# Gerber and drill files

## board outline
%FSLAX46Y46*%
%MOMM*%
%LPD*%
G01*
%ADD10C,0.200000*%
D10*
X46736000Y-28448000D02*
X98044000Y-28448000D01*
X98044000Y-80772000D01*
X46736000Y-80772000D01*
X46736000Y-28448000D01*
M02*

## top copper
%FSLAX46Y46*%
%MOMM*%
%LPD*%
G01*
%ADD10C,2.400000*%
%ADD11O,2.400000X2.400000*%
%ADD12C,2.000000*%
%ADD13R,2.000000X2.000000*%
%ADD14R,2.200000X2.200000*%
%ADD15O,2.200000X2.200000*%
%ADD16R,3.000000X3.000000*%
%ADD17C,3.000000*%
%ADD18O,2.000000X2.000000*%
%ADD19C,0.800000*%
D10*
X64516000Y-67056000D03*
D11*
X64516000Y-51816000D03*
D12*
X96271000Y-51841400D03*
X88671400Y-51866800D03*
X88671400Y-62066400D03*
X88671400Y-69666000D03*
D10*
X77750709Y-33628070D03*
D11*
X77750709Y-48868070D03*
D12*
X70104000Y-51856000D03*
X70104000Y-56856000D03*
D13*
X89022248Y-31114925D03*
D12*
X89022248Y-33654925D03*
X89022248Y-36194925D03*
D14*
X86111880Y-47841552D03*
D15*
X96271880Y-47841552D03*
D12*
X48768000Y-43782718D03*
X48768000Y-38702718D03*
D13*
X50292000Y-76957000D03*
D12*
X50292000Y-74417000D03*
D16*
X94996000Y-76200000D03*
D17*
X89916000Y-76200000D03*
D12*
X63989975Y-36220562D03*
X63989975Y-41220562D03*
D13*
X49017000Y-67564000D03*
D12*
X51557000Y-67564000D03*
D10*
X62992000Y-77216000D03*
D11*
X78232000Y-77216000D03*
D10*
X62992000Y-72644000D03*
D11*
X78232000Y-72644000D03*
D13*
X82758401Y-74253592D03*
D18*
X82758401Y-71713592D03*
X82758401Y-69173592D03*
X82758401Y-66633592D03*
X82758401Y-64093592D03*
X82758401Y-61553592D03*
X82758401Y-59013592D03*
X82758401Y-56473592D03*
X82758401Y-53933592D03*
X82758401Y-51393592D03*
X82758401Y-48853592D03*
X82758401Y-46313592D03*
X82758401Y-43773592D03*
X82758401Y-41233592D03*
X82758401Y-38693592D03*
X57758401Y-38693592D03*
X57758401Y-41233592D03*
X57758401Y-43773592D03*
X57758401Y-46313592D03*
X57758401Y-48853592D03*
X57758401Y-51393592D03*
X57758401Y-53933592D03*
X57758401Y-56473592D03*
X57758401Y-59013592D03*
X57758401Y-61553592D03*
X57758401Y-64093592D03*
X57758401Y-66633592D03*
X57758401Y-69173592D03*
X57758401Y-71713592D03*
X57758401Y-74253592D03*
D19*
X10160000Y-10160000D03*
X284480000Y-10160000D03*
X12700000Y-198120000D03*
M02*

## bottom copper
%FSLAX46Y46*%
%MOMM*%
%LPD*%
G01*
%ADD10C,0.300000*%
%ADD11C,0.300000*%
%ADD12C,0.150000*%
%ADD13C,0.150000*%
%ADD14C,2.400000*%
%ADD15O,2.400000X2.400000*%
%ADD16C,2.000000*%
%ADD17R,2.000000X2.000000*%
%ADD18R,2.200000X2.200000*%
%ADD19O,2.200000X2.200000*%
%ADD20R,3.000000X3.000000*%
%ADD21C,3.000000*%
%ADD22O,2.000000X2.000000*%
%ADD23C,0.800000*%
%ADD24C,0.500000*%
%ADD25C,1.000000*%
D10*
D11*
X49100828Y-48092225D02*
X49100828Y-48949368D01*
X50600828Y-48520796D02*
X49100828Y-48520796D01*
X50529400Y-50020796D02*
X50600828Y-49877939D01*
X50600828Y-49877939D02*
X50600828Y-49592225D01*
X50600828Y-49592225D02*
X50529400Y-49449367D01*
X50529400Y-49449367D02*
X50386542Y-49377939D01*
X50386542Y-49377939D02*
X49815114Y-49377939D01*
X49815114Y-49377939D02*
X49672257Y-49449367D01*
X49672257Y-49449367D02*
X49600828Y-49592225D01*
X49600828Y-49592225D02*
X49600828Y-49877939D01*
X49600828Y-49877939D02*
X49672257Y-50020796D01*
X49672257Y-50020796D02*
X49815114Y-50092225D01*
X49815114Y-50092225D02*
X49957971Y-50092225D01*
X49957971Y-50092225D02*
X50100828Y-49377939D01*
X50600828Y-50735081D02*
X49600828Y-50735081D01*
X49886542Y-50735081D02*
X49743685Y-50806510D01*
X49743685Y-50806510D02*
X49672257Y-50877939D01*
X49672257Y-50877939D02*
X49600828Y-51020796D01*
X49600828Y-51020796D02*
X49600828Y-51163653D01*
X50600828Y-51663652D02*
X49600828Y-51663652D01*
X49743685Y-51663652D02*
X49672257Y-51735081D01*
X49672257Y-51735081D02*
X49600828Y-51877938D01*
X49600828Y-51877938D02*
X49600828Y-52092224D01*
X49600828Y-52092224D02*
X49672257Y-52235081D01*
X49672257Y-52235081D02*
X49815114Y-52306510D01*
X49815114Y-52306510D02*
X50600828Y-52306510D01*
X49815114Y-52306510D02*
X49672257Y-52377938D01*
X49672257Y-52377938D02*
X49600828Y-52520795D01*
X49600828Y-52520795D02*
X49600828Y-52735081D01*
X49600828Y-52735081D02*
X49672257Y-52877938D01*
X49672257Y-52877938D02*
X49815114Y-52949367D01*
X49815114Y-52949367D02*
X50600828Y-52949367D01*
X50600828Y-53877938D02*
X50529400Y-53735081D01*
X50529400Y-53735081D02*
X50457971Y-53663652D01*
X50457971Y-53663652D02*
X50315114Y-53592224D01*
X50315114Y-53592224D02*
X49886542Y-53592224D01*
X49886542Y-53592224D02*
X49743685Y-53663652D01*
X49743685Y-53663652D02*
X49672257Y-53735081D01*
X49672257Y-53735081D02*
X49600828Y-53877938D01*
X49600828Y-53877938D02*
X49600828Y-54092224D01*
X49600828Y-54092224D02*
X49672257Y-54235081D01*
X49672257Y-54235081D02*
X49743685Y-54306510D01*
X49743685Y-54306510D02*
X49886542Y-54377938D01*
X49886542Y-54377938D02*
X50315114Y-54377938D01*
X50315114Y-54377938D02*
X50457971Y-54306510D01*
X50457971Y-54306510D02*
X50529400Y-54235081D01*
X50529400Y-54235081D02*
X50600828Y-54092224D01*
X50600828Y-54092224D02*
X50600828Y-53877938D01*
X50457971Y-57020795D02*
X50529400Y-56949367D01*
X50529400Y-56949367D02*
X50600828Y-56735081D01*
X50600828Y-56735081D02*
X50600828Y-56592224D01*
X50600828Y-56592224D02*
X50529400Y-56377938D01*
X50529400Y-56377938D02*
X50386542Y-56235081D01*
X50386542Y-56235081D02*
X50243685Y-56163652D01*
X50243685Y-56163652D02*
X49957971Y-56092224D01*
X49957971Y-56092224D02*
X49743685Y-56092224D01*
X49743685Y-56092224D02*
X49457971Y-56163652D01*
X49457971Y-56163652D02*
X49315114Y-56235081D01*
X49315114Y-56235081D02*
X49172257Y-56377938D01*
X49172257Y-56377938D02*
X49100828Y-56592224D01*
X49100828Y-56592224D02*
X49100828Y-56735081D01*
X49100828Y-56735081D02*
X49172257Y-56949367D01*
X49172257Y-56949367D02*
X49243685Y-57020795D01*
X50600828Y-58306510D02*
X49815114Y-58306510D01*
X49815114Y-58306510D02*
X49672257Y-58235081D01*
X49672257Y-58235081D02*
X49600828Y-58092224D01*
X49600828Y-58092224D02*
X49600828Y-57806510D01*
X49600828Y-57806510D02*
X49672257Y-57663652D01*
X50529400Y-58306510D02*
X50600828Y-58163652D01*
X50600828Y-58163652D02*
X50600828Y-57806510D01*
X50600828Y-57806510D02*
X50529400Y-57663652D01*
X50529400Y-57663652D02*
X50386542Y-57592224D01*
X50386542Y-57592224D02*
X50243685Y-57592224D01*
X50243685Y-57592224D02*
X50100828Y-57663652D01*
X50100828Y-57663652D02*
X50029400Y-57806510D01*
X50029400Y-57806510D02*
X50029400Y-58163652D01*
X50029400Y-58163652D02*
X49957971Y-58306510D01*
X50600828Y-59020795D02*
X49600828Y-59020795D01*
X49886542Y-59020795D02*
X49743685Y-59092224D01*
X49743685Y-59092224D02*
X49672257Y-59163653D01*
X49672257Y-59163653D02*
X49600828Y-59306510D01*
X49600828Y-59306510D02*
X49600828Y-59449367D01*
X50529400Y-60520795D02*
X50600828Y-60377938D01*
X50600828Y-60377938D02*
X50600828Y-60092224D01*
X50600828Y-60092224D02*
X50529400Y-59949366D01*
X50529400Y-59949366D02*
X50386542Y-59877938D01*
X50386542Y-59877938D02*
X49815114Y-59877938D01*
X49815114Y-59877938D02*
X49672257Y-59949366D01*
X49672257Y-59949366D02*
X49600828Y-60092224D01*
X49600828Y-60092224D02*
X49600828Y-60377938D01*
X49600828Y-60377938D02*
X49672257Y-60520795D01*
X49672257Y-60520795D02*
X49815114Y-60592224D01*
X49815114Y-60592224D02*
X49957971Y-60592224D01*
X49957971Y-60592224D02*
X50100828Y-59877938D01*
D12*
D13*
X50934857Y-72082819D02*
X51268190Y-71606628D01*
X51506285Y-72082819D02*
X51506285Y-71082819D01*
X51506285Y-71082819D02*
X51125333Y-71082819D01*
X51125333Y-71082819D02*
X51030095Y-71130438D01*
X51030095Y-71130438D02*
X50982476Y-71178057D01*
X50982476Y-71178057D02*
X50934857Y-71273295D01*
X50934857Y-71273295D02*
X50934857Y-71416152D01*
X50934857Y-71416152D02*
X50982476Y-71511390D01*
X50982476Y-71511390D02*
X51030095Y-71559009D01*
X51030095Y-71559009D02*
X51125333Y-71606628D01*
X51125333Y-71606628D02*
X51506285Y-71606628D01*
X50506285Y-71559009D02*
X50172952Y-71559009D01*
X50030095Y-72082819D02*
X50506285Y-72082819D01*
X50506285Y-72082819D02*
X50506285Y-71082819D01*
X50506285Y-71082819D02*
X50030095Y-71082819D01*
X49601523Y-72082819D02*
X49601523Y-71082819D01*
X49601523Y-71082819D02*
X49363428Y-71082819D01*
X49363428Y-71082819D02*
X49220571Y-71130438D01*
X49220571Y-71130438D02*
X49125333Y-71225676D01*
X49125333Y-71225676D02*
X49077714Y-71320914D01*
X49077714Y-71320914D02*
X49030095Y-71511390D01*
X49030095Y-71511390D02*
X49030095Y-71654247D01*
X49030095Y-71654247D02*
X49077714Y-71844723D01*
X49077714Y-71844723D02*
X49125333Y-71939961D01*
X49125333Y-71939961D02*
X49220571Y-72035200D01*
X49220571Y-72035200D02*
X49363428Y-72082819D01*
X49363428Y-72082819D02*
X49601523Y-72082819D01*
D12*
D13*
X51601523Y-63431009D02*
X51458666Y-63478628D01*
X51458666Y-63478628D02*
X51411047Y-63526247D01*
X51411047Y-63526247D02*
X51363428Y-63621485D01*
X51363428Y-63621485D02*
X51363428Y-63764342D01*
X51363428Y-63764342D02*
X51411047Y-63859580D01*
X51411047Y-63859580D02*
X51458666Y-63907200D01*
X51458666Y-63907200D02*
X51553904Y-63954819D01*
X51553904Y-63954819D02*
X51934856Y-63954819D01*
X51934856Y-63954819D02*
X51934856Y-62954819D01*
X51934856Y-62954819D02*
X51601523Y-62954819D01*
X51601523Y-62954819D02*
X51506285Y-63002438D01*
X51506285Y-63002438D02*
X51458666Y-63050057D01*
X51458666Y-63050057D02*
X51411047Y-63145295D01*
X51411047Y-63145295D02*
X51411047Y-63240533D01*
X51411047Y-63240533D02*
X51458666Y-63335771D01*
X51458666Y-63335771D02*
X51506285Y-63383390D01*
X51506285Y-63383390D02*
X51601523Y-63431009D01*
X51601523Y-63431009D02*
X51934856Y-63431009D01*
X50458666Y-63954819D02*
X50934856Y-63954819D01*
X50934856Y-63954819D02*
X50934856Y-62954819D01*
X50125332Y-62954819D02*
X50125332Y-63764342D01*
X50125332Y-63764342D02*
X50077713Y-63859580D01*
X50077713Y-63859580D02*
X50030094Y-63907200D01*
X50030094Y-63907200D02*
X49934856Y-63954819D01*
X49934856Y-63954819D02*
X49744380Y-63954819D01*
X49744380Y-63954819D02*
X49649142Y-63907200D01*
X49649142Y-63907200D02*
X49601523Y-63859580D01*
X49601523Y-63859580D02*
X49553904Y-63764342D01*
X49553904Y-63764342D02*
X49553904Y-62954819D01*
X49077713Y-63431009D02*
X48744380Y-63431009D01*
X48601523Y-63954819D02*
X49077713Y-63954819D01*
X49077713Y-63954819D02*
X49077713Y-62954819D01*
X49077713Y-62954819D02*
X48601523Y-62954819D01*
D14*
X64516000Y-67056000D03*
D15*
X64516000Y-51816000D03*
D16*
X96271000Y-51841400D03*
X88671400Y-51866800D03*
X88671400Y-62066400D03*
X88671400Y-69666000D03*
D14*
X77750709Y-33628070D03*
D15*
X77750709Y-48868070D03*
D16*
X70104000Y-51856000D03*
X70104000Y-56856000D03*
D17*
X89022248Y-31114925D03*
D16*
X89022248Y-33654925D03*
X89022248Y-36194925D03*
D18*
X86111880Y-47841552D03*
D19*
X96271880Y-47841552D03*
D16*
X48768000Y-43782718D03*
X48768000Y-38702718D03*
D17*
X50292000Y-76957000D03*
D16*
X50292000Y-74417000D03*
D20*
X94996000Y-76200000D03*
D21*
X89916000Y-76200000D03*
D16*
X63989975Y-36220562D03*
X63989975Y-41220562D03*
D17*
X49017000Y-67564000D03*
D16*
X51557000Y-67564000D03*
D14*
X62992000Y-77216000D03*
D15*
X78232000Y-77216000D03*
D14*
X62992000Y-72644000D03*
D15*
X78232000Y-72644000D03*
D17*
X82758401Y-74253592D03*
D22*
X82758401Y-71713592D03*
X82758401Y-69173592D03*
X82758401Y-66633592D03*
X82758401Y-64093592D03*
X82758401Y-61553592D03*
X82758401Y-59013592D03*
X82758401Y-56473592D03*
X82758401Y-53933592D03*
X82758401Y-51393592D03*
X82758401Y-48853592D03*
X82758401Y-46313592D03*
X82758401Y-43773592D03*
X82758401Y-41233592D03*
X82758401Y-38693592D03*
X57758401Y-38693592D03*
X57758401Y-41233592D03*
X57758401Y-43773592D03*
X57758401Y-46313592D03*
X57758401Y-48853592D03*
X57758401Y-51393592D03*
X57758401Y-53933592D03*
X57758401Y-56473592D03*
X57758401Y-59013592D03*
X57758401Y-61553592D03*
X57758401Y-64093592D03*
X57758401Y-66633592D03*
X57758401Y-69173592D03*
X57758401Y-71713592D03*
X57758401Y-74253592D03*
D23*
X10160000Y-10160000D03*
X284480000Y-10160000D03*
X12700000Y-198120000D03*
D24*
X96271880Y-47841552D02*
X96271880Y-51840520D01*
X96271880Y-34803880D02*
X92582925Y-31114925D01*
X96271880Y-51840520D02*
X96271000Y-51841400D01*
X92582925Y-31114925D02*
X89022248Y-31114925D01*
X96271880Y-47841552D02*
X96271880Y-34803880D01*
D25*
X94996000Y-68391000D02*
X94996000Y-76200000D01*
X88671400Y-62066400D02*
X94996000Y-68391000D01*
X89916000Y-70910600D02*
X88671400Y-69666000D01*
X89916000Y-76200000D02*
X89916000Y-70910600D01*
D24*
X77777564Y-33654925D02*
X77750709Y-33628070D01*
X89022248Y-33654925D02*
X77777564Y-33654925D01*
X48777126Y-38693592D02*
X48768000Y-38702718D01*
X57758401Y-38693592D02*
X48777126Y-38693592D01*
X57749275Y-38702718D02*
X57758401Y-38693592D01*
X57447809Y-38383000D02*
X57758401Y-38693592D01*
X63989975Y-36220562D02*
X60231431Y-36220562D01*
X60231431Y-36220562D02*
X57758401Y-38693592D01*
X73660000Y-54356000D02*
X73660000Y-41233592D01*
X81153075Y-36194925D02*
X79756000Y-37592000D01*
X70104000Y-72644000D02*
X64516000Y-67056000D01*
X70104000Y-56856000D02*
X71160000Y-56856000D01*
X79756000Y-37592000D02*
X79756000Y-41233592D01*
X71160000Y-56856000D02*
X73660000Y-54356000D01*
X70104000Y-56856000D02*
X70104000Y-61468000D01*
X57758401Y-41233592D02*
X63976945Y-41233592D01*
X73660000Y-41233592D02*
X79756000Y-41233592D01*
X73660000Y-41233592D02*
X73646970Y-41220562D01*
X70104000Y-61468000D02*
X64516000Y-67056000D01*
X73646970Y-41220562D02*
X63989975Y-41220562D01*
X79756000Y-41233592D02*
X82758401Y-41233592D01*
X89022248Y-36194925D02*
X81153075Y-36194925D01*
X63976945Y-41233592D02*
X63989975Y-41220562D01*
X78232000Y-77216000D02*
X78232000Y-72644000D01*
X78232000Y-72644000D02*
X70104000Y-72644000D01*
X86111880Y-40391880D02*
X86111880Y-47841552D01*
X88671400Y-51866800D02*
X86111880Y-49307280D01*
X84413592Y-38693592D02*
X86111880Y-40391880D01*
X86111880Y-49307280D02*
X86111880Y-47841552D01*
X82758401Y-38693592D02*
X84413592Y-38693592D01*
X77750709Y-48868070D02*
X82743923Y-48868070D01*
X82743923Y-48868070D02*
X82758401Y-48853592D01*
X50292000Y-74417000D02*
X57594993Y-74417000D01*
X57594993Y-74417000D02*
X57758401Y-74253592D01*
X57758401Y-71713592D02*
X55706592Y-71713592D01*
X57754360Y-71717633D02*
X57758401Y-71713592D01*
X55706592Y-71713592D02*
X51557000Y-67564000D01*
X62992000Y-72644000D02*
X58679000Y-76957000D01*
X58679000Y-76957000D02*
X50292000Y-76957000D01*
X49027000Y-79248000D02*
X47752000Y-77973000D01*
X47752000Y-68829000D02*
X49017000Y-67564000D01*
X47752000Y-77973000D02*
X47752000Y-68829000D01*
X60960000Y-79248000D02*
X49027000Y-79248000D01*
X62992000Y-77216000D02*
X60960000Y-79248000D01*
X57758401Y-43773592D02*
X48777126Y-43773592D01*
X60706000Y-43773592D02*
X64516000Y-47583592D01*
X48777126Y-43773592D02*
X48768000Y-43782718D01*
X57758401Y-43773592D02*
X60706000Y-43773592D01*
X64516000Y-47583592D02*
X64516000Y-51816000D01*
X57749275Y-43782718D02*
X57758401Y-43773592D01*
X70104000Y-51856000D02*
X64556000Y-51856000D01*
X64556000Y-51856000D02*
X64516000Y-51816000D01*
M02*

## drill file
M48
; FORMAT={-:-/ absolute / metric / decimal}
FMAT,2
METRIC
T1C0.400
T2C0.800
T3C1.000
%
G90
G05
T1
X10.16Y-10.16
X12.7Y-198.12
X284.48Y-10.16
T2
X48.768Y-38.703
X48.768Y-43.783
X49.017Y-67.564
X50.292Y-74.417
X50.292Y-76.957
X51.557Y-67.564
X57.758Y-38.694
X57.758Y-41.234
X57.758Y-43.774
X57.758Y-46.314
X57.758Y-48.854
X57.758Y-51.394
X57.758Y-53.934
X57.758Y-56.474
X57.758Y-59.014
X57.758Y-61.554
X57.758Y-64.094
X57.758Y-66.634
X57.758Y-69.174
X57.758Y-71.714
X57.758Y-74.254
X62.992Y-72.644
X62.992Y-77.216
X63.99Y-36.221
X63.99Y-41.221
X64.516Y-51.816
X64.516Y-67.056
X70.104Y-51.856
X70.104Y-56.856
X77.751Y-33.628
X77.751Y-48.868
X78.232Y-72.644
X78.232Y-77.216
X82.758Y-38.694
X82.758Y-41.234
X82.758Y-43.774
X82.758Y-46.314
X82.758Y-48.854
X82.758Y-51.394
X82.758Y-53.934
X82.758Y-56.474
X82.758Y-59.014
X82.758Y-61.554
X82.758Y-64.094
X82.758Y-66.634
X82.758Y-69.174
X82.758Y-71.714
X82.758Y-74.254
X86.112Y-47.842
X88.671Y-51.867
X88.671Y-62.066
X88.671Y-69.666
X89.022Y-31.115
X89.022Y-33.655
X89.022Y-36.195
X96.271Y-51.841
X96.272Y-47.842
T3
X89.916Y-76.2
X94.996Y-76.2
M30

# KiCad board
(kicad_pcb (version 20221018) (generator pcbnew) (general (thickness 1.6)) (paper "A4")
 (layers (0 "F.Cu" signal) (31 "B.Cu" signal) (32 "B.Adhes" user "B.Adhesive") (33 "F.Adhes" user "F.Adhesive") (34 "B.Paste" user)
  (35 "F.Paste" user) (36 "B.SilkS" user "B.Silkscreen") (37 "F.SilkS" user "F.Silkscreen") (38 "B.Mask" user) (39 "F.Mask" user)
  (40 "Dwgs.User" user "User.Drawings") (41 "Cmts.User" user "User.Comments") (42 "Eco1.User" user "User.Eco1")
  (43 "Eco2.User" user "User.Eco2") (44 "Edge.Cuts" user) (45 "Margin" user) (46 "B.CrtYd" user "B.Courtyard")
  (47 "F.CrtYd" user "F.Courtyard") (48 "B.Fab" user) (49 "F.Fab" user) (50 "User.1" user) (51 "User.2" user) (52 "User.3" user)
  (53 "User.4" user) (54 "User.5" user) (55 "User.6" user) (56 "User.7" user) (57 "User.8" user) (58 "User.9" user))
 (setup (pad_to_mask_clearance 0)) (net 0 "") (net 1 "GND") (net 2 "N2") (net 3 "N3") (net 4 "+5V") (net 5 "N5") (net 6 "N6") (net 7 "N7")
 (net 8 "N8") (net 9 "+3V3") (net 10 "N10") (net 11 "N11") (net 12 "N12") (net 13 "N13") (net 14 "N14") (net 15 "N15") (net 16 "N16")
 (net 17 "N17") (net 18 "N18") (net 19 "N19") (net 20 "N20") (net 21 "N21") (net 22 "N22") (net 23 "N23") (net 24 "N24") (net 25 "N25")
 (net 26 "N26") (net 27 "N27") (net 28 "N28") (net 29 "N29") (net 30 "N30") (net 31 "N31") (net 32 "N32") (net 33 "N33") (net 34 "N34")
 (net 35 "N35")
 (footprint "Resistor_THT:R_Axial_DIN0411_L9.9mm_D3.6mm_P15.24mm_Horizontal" (layer "F.Cu") (at 64.516 67.056 90)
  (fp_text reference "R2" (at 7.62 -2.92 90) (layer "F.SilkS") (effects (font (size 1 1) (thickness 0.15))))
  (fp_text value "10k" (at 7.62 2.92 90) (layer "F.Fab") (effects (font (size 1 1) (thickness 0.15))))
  (pad "1" thru_hole circle (at 0 0 90) (size 2.4 2.4) (drill 0.8) (layers "*.Cu" "*.Mask") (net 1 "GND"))
  (pad "2" thru_hole oval (at 15.24 0 90) (size 2.4 2.4) (drill 0.8) (layers "*.Cu" "*.Mask") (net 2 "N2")))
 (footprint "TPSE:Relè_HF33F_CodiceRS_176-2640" (layer "F.Cu") (at 92.456 60.96 -90)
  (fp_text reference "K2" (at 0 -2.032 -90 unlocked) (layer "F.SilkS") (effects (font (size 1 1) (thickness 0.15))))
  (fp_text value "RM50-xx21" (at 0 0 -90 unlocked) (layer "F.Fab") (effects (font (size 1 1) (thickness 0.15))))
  (pad "1" thru_hole circle (at -9.1186 -3.815 270) (size 2 2) (drill 0.8) (layers "*.Cu" "*.Mask") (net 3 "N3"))
  (pad "2" thru_hole circle (at -9.0932 3.7846 270) (size 2 2) (drill 0.8) (layers "*.Cu" "*.Mask") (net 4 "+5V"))
  (pad "3" thru_hole circle (at 1.1064 3.7846 270) (size 2 2) (drill 0.8) (layers "*.Cu" "*.Mask") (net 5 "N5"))
  (pad "4" thru_hole circle (at 8.706 3.7846 270) (size 2 2) (drill 0.8) (layers "*.Cu" "*.Mask") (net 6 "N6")))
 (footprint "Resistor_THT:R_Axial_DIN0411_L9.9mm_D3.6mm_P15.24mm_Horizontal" (layer "F.Cu") (at 77.750709 33.62807 -90)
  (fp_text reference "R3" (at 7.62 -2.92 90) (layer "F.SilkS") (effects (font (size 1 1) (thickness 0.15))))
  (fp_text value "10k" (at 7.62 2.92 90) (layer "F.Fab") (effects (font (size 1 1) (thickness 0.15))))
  (pad "1" thru_hole circle (at 0 0 270) (size 2.4 2.4) (drill 0.8) (layers "*.Cu" "*.Mask") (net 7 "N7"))
  (pad "2" thru_hole oval (at 15.24 0 270) (size 2.4 2.4) (drill 0.8) (layers "*.Cu" "*.Mask") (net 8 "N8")))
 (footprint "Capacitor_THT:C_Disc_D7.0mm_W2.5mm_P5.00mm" (layer "F.Cu") (at 70.104 51.856 -90)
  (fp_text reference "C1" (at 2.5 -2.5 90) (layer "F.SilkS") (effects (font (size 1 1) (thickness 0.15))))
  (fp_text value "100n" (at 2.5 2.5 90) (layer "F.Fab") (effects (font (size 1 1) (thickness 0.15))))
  (pad "1" thru_hole circle (at 0 0 270) (size 2 2) (drill 0.8) (layers "*.Cu" "*.Mask") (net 2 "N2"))
  (pad "2" thru_hole circle (at 5 0 270) (size 2 2) (drill 0.8) (layers "*.Cu" "*.Mask") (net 1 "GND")))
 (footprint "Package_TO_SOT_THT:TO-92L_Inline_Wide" (layer "F.Cu") (at 89.022248 31.114925 -90)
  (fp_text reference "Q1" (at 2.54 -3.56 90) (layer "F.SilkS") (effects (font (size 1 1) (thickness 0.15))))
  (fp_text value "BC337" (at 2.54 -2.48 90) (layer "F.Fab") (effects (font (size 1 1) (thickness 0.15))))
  (pad "1" thru_hole rect (at 0 0 270) (size 2 2) (drill 0.8) (layers "*.Cu" "*.Mask") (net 3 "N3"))
  (pad "2" thru_hole circle (at 2.54 0 270) (size 2 2) (drill 0.8) (layers "*.Cu" "*.Mask") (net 7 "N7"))
  (pad "3" thru_hole circle (at 5.08 0 270) (size 2 2) (drill 0.8) (layers "*.Cu" "*.Mask") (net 1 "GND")))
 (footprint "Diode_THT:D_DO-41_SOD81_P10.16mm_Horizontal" (layer "F.Cu") (at 86.11188 47.841552)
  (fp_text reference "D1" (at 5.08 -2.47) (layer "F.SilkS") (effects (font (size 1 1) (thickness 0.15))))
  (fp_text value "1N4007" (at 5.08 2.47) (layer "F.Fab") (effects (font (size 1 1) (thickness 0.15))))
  (pad "1" thru_hole rect (at 0 0) (size 2.2 2.2) (drill 0.8) (layers "*.Cu" "*.Mask") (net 4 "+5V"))
  (pad "2" thru_hole oval (at 10.16 0) (size 2.2 2.2) (drill 0.8) (layers "*.Cu" "*.Mask") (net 3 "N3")))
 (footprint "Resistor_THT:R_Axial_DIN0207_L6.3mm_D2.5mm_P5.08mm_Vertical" (layer "F.Cu") (at 48.768 43.782718 90)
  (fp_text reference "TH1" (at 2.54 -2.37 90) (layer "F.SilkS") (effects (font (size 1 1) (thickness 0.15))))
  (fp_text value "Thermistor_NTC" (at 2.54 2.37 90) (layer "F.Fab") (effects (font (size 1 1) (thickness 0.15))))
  (pad "1" thru_hole circle (at 0 0 90) (size 2 2) (drill 0.8) (layers "*.Cu" "*.Mask") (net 2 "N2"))
  (pad "2" thru_hole circle (at 5.08 0 90) (size 2 2) (drill 0.8) (layers "*.Cu" "*.Mask") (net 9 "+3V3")))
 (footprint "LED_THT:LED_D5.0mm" (layer "F.Cu") (at 50.292 76.957 90)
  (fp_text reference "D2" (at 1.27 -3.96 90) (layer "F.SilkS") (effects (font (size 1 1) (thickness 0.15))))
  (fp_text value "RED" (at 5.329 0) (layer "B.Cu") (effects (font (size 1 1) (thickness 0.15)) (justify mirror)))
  (pad "1" thru_hole rect (at 0 0 90) (size 2 2) (drill 0.8) (layers "*.Cu" "*.Mask") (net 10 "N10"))
  (pad "2" thru_hole circle (at 2.54 0 90) (size 2 2) (drill 0.8) (layers "*.Cu" "*.Mask") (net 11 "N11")))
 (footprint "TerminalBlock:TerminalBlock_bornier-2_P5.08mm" (layer "F.Cu") (at 94.996 76.2 180)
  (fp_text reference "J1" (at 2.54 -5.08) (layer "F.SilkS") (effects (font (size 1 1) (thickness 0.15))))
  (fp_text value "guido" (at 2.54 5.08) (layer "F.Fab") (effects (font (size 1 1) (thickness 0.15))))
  (pad "1" thru_hole rect (at 0 0 180) (size 3 3) (drill 1) (layers "*.Cu" "*.Mask") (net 5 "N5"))
  (pad "2" thru_hole circle (at 5.08 0 180) (size 3 3) (drill 1) (layers "*.Cu" "*.Mask") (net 6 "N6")))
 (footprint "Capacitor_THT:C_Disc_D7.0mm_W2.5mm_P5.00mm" (layer "F.Cu") (at 63.989975 36.220562 -90)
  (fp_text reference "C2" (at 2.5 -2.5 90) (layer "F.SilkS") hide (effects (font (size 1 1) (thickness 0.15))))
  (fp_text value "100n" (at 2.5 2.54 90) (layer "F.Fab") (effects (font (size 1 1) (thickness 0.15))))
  (pad "1" thru_hole circle (at 0 0 270) (size 2 2) (drill 0.8) (layers "*.Cu" "*.Mask") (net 9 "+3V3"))
  (pad "2" thru_hole circle (at 5 0 270) (size 2 2) (drill 0.8) (layers "*.Cu" "*.Mask") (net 1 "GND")))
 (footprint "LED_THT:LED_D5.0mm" (layer "F.Cu") (at 49.017 67.564)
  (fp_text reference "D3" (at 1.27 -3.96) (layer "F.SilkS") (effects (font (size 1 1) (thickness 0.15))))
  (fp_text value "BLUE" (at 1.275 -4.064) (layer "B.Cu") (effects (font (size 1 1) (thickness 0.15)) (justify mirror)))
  (pad "1" thru_hole rect (at 0 0) (size 2 2) (drill 0.8) (layers "*.Cu" "*.Mask") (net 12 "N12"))
  (pad "2" thru_hole circle (at 2.54 0) (size 2 2) (drill 0.8) (layers "*.Cu" "*.Mask") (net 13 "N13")))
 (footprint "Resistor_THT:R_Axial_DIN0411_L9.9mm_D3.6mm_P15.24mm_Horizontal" (layer "F.Cu") (at 62.992 77.216)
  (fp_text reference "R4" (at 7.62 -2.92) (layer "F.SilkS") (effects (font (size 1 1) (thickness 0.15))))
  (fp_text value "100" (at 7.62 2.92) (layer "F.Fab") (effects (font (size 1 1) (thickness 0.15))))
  (pad "1" thru_hole circle (at 0 0) (size 2.4 2.4) (drill 0.8) (layers "*.Cu" "*.Mask") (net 12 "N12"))
  (pad "2" thru_hole oval (at 15.24 0) (size 2.4 2.4) (drill 0.8) (layers "*.Cu" "*.Mask") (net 1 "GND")))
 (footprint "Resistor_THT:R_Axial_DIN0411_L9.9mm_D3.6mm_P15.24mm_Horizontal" (layer "F.Cu") (at 62.992 72.644)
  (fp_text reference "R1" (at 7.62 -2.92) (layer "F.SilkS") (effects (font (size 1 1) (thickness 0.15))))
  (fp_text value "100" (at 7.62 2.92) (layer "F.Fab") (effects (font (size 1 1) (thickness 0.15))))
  (pad "1" thru_hole circle (at 0 0) (size 2.4 2.4) (drill 0.8) (layers "*.Cu" "*.Mask") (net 10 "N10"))
  (pad "2" thru_hole oval (at 15.24 0) (size 2.4 2.4) (drill 0.8) (layers "*.Cu" "*.Mask") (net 1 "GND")))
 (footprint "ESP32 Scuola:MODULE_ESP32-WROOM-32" (layer "F.Cu") (at 70.258401 53.953592 180)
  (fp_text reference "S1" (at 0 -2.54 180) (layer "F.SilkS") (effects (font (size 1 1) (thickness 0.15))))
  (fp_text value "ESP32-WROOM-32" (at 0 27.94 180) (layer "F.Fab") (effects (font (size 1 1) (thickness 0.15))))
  (pad "1" thru_hole rect (at -12.5 -20.3 180) (size 2 2) (drill 0.8) (layers "*.Cu" "*.Mask") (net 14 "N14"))
  (pad "2" thru_hole oval (at -12.5 -17.76 180) (size 2 2) (drill 0.8) (layers "*.Cu" "*.Mask") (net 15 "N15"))
  (pad "3" thru_hole oval (at -12.5 -15.22 180) (size 2 2) (drill 0.8) (layers "*.Cu" "*.Mask") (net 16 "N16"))
  (pad "4" thru_hole oval (at -12.5 -12.68 180) (size 2 2) (drill 0.8) (layers "*.Cu" "*.Mask") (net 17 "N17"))
  (pad "5" thru_hole oval (at -12.5 -10.14 180) (size 2 2) (drill 0.8) (layers "*.Cu" "*.Mask") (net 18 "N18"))
  (pad "6" thru_hole oval (at -12.5 -7.6 180) (size 2 2) (drill 0.8) (layers "*.Cu" "*.Mask") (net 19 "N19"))
  (pad "7" thru_hole oval (at -12.5 -5.06 180) (size 2 2) (drill 0.8) (layers "*.Cu" "*.Mask") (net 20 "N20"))
  (pad "8" thru_hole oval (at -12.5 -2.52 180) (size 2 2) (drill 0.8) (layers "*.Cu" "*.Mask") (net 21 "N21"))
  (pad "9" thru_hole oval (at -12.5 0.02 180) (size 2 2) (drill 0.8) (layers "*.Cu" "*.Mask") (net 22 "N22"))
  (pad "10" thru_hole oval (at -12.5 2.56 180) (size 2 2) (drill 0.8) (layers "*.Cu" "*.Mask") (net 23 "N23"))
  (pad "11" thru_hole oval (at -12.5 5.1 180) (size 2 2) (drill 0.8) (layers "*.Cu" "*.Mask") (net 8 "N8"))
  (pad "12" thru_hole oval (at -12.5 7.64 180) (size 2 2) (drill 0.8) (layers "*.Cu" "*.Mask") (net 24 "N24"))
  (pad "13" thru_hole oval (at -12.5 10.18 180) (size 2 2) (drill 0.8) (layers "*.Cu" "*.Mask") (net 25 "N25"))
  (pad "14" thru_hole oval (at -12.5 12.72 180) (size 2 2) (drill 0.8) (layers "*.Cu" "*.Mask") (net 1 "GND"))
  (pad "15" thru_hole oval (at -12.5 15.26 180) (size 2 2) (drill 0.8) (layers "*.Cu" "*.Mask") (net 4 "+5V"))
  (pad "16" thru_hole oval (at 12.5 15.26 180) (size 2 2) (drill 0.8) (layers "*.Cu" "*.Mask") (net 9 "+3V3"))
  (pad "17" thru_hole oval (at 12.5 12.72 180) (size 2 2) (drill 0.8) (layers "*.Cu" "*.Mask") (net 1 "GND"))
  (pad "18" thru_hole oval (at 12.5 10.18 180) (size 2 2) (drill 0.8) (layers "*.Cu" "*.Mask") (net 2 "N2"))
  (pad "19" thru_hole oval (at 12.5 7.64 180) (size 2 2) (drill 0.8) (layers "*.Cu" "*.Mask") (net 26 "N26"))
  (pad "20" thru_hole oval (at 12.5 5.1 180) (size 2 2) (drill 0.8) (layers "*.Cu" "*.Mask") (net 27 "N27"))
  (pad "21" thru_hole oval (at 12.5 2.56 180) (size 2 2) (drill 0.8) (layers "*.Cu" "*.Mask") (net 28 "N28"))
  (pad "22" thru_hole oval (at 12.5 0.02 180) (size 2 2) (drill 0.8) (layers "*.Cu" "*.Mask") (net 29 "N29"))
  (pad "23" thru_hole oval (at 12.5 -2.52 180) (size 2 2) (drill 0.8) (layers "*.Cu" "*.Mask") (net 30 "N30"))
  (pad "24" thru_hole oval (at 12.5 -5.06 180) (size 2 2) (drill 0.8) (layers "*.Cu" "*.Mask") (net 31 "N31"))
  (pad "25" thru_hole oval (at 12.5 -7.6 180) (size 2 2) (drill 0.8) (layers "*.Cu" "*.Mask") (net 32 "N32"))
  (pad "26" thru_hole oval (at 12.5 -10.14 180) (size 2 2) (drill 0.8) (layers "*.Cu" "*.Mask") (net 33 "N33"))
  (pad "27" thru_hole oval (at 12.5 -12.68 180) (size 2 2) (drill 0.8) (layers "*.Cu" "*.Mask") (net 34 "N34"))
  (pad "28" thru_hole oval (at 12.5 -15.22 180) (size 2 2) (drill 0.8) (layers "*.Cu" "*.Mask") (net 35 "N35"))
  (pad "29" thru_hole oval (at 12.5 -17.76 180) (size 2 2) (drill 0.8) (layers "*.Cu" "*.Mask") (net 13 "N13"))
  (pad "30" thru_hole oval (at 12.5 -20.3 180) (size 2 2) (drill 0.8) (layers "*.Cu" "*.Mask") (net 11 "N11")))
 (gr_rect (start 46.736 28.448) (end 98.044 80.772) (stroke (width 0.2) (type default)) (fill none) (layer "Edge.Cuts"))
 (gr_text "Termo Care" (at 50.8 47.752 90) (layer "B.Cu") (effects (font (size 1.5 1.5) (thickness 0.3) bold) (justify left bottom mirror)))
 (via (at 10.16 10.16) (size 0.8) (drill 0.4) (layers "F.Cu" "B.Cu") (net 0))
 (via (at 284.48 10.16) (size 0.8) (drill 0.4) (layers "F.Cu" "B.Cu") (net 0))
 (via (at 12.7 198.12) (size 0.8) (drill 0.4) (layers "F.Cu" "B.Cu") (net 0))
 (segment (start 96.27188 47.841552) (end 96.27188 51.84052) (width 0.5) (layer "B.Cu") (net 3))
 (segment (start 96.27188 34.80388) (end 92.582925 31.114925) (width 0.5) (layer "B.Cu") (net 3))
 (segment (start 96.27188 51.84052) (end 96.271 51.8414) (width 0.5) (layer "B.Cu") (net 3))
 (segment (start 92.582925 31.114925) (end 89.022248 31.114925) (width 0.5) (layer "B.Cu") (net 3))
 (segment (start 96.27188 47.841552) (end 96.27188 34.80388) (width 0.5) (layer "B.Cu") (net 3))
 (segment (start 94.996 68.391) (end 94.996 76.2) (width 1) (layer "B.Cu") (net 5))
 (segment (start 88.6714 62.0664) (end 94.996 68.391) (width 1) (layer "B.Cu") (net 5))
 (segment (start 89.916 70.9106) (end 88.6714 69.666) (width 1) (layer "B.Cu") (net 6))
 (segment (start 89.916 76.2) (end 89.916 70.9106) (width 1) (layer "B.Cu") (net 6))
 (segment (start 77.777564 33.654925) (end 77.750709 33.62807) (width 0.5) (layer "B.Cu") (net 7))
 (segment (start 89.022248 33.654925) (end 77.777564 33.654925) (width 0.5) (layer "B.Cu") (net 7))
 (segment (start 48.777126 38.693592) (end 48.768 38.702718) (width 0.5) (layer "B.Cu") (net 9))
 (segment (start 57.758401 38.693592) (end 48.777126 38.693592) (width 0.5) (layer "B.Cu") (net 9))
 (segment (start 57.749275 38.702718) (end 57.758401 38.693592) (width 0.5) (layer "B.Cu") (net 9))
 (segment (start 57.447809 38.383) (end 57.758401 38.693592) (width 0.5) (layer "B.Cu") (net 9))
 (segment (start 63.989975 36.220562) (end 60.231431 36.220562) (width 0.5) (layer "B.Cu") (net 9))
 (segment (start 60.231431 36.220562) (end 57.758401 38.693592) (width 0.5) (layer "B.Cu") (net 9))
 (segment (start 73.66 54.356) (end 73.66 41.233592) (width 0.5) (layer "B.Cu") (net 1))
 (segment (start 81.153075 36.194925) (end 79.756 37.592) (width 0.5) (layer "B.Cu") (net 1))
 (segment (start 70.104 72.644) (end 64.516 67.056) (width 0.5) (layer "B.Cu") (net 1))
 (segment (start 70.104 56.856) (end 71.16 56.856) (width 0.5) (layer "B.Cu") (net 1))
 (segment (start 79.756 37.592) (end 79.756 41.233592) (width 0.5) (layer "B.Cu") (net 1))
 (segment (start 71.16 56.856) (end 73.66 54.356) (width 0.5) (layer "B.Cu") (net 1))
 (segment (start 70.104 56.856) (end 70.104 61.468) (width 0.5) (layer "B.Cu") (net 1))
 (segment (start 57.758401 41.233592) (end 63.976945 41.233592) (width 0.5) (layer "B.Cu") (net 1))
 (segment (start 73.66 41.233592) (end 79.756 41.233592) (width 0.5) (layer "B.Cu") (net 1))
 (segment (start 73.66 41.233592) (end 73.64697 41.220562) (width 0.5) (layer "B.Cu") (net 1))
 (segment (start 70.104 61.468) (end 64.516 67.056) (width 0.5) (layer "B.Cu") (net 1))
 (segment (start 73.64697 41.220562) (end 63.989975 41.220562) (width 0.5) (layer "B.Cu") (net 1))
 (segment (start 79.756 41.233592) (end 82.758401 41.233592) (width 0.5) (layer "B.Cu") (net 1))
 (segment (start 89.022248 36.194925) (end 81.153075 36.194925) (width 0.5) (layer "B.Cu") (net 1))
 (segment (start 63.976945 41.233592) (end 63.989975 41.220562) (width 0.5) (layer "B.Cu") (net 1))
 (segment (start 78.232 77.216) (end 78.232 72.644) (width 0.5) (layer "B.Cu") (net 1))
 (segment (start 78.232 72.644) (end 70.104 72.644) (width 0.5) (layer "B.Cu") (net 1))
 (segment (start 86.11188 40.39188) (end 86.11188 47.841552) (width 0.5) (layer "B.Cu") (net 4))
 (segment (start 88.6714 51.8668) (end 86.11188 49.30728) (width 0.5) (layer "B.Cu") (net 4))
 (segment (start 84.413592 38.693592) (end 86.11188 40.39188) (width 0.5) (layer "B.Cu") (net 4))
 (segment (start 86.11188 49.30728) (end 86.11188 47.841552) (width 0.5) (layer "B.Cu") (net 4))
 (segment (start 82.758401 38.693592) (end 84.413592 38.693592) (width 0.5) (layer "B.Cu") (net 4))
 (segment (start 77.750709 48.86807) (end 82.743923 48.86807) (width 0.5) (layer "B.Cu") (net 8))
 (segment (start 82.743923 48.86807) (end 82.758401 48.853592) (width 0.5) (layer "B.Cu") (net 8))
 (segment (start 50.292 74.417) (end 57.594993 74.417) (width 0.5) (layer "B.Cu") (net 11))
 (segment (start 57.594993 74.417) (end 57.758401 74.253592) (width 0.5) (layer "B.Cu") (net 11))
 (segment (start 57.758401 71.713592) (end 55.706592 71.713592) (width 0.5) (layer "B.Cu") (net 13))
 (segment (start 57.75436 71.717633) (end 57.758401 71.713592) (width 0.5) (layer "B.Cu") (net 13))
 (segment (start 55.706592 71.713592) (end 51.557 67.564) (width 0.5) (layer "B.Cu") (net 13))
 (segment (start 62.992 72.644) (end 58.679 76.957) (width 0.5) (layer "B.Cu") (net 10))
 (segment (start 58.679 76.957) (end 50.292 76.957) (width 0.5) (layer "B.Cu") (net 10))
 (segment (start 49.027 79.248) (end 47.752 77.973) (width 0.5) (layer "B.Cu") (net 12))
 (segment (start 47.752 68.829) (end 49.017 67.564) (width 0.5) (layer "B.Cu") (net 12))
 (segment (start 47.752 77.973) (end 47.752 68.829) (width 0.5) (layer "B.Cu") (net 12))
 (segment (start 60.96 79.248) (end 49.027 79.248) (width 0.5) (layer "B.Cu") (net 12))
 (segment (start 62.992 77.216) (end 60.96 79.248) (width 0.5) (layer "B.Cu") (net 12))
 (segment (start 57.758401 43.773592) (end 48.777126 43.773592) (width 0.5) (layer "B.Cu") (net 2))
 (segment (start 60.706 43.773592) (end 64.516 47.583592) (width 0.5) (layer "B.Cu") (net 2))
 (segment (start 48.777126 43.773592) (end 48.768 43.782718) (width 0.5) (layer "B.Cu") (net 2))
 (segment (start 57.758401 43.773592) (end 60.706 43.773592) (width 0.5) (layer "B.Cu") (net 2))
 (segment (start 64.516 47.583592) (end 64.516 51.816) (width 0.5) (layer "B.Cu") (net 2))
 (segment (start 57.749275 43.782718) (end 57.758401 43.773592) (width 0.5) (layer "B.Cu") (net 2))
 (segment (start 70.104 51.856) (end 64.556 51.856) (width 0.5) (layer "B.Cu") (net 2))
 (segment (start 64.556 51.856) (end 64.516 51.816) (width 0.5) (layer "B.Cu") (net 2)))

